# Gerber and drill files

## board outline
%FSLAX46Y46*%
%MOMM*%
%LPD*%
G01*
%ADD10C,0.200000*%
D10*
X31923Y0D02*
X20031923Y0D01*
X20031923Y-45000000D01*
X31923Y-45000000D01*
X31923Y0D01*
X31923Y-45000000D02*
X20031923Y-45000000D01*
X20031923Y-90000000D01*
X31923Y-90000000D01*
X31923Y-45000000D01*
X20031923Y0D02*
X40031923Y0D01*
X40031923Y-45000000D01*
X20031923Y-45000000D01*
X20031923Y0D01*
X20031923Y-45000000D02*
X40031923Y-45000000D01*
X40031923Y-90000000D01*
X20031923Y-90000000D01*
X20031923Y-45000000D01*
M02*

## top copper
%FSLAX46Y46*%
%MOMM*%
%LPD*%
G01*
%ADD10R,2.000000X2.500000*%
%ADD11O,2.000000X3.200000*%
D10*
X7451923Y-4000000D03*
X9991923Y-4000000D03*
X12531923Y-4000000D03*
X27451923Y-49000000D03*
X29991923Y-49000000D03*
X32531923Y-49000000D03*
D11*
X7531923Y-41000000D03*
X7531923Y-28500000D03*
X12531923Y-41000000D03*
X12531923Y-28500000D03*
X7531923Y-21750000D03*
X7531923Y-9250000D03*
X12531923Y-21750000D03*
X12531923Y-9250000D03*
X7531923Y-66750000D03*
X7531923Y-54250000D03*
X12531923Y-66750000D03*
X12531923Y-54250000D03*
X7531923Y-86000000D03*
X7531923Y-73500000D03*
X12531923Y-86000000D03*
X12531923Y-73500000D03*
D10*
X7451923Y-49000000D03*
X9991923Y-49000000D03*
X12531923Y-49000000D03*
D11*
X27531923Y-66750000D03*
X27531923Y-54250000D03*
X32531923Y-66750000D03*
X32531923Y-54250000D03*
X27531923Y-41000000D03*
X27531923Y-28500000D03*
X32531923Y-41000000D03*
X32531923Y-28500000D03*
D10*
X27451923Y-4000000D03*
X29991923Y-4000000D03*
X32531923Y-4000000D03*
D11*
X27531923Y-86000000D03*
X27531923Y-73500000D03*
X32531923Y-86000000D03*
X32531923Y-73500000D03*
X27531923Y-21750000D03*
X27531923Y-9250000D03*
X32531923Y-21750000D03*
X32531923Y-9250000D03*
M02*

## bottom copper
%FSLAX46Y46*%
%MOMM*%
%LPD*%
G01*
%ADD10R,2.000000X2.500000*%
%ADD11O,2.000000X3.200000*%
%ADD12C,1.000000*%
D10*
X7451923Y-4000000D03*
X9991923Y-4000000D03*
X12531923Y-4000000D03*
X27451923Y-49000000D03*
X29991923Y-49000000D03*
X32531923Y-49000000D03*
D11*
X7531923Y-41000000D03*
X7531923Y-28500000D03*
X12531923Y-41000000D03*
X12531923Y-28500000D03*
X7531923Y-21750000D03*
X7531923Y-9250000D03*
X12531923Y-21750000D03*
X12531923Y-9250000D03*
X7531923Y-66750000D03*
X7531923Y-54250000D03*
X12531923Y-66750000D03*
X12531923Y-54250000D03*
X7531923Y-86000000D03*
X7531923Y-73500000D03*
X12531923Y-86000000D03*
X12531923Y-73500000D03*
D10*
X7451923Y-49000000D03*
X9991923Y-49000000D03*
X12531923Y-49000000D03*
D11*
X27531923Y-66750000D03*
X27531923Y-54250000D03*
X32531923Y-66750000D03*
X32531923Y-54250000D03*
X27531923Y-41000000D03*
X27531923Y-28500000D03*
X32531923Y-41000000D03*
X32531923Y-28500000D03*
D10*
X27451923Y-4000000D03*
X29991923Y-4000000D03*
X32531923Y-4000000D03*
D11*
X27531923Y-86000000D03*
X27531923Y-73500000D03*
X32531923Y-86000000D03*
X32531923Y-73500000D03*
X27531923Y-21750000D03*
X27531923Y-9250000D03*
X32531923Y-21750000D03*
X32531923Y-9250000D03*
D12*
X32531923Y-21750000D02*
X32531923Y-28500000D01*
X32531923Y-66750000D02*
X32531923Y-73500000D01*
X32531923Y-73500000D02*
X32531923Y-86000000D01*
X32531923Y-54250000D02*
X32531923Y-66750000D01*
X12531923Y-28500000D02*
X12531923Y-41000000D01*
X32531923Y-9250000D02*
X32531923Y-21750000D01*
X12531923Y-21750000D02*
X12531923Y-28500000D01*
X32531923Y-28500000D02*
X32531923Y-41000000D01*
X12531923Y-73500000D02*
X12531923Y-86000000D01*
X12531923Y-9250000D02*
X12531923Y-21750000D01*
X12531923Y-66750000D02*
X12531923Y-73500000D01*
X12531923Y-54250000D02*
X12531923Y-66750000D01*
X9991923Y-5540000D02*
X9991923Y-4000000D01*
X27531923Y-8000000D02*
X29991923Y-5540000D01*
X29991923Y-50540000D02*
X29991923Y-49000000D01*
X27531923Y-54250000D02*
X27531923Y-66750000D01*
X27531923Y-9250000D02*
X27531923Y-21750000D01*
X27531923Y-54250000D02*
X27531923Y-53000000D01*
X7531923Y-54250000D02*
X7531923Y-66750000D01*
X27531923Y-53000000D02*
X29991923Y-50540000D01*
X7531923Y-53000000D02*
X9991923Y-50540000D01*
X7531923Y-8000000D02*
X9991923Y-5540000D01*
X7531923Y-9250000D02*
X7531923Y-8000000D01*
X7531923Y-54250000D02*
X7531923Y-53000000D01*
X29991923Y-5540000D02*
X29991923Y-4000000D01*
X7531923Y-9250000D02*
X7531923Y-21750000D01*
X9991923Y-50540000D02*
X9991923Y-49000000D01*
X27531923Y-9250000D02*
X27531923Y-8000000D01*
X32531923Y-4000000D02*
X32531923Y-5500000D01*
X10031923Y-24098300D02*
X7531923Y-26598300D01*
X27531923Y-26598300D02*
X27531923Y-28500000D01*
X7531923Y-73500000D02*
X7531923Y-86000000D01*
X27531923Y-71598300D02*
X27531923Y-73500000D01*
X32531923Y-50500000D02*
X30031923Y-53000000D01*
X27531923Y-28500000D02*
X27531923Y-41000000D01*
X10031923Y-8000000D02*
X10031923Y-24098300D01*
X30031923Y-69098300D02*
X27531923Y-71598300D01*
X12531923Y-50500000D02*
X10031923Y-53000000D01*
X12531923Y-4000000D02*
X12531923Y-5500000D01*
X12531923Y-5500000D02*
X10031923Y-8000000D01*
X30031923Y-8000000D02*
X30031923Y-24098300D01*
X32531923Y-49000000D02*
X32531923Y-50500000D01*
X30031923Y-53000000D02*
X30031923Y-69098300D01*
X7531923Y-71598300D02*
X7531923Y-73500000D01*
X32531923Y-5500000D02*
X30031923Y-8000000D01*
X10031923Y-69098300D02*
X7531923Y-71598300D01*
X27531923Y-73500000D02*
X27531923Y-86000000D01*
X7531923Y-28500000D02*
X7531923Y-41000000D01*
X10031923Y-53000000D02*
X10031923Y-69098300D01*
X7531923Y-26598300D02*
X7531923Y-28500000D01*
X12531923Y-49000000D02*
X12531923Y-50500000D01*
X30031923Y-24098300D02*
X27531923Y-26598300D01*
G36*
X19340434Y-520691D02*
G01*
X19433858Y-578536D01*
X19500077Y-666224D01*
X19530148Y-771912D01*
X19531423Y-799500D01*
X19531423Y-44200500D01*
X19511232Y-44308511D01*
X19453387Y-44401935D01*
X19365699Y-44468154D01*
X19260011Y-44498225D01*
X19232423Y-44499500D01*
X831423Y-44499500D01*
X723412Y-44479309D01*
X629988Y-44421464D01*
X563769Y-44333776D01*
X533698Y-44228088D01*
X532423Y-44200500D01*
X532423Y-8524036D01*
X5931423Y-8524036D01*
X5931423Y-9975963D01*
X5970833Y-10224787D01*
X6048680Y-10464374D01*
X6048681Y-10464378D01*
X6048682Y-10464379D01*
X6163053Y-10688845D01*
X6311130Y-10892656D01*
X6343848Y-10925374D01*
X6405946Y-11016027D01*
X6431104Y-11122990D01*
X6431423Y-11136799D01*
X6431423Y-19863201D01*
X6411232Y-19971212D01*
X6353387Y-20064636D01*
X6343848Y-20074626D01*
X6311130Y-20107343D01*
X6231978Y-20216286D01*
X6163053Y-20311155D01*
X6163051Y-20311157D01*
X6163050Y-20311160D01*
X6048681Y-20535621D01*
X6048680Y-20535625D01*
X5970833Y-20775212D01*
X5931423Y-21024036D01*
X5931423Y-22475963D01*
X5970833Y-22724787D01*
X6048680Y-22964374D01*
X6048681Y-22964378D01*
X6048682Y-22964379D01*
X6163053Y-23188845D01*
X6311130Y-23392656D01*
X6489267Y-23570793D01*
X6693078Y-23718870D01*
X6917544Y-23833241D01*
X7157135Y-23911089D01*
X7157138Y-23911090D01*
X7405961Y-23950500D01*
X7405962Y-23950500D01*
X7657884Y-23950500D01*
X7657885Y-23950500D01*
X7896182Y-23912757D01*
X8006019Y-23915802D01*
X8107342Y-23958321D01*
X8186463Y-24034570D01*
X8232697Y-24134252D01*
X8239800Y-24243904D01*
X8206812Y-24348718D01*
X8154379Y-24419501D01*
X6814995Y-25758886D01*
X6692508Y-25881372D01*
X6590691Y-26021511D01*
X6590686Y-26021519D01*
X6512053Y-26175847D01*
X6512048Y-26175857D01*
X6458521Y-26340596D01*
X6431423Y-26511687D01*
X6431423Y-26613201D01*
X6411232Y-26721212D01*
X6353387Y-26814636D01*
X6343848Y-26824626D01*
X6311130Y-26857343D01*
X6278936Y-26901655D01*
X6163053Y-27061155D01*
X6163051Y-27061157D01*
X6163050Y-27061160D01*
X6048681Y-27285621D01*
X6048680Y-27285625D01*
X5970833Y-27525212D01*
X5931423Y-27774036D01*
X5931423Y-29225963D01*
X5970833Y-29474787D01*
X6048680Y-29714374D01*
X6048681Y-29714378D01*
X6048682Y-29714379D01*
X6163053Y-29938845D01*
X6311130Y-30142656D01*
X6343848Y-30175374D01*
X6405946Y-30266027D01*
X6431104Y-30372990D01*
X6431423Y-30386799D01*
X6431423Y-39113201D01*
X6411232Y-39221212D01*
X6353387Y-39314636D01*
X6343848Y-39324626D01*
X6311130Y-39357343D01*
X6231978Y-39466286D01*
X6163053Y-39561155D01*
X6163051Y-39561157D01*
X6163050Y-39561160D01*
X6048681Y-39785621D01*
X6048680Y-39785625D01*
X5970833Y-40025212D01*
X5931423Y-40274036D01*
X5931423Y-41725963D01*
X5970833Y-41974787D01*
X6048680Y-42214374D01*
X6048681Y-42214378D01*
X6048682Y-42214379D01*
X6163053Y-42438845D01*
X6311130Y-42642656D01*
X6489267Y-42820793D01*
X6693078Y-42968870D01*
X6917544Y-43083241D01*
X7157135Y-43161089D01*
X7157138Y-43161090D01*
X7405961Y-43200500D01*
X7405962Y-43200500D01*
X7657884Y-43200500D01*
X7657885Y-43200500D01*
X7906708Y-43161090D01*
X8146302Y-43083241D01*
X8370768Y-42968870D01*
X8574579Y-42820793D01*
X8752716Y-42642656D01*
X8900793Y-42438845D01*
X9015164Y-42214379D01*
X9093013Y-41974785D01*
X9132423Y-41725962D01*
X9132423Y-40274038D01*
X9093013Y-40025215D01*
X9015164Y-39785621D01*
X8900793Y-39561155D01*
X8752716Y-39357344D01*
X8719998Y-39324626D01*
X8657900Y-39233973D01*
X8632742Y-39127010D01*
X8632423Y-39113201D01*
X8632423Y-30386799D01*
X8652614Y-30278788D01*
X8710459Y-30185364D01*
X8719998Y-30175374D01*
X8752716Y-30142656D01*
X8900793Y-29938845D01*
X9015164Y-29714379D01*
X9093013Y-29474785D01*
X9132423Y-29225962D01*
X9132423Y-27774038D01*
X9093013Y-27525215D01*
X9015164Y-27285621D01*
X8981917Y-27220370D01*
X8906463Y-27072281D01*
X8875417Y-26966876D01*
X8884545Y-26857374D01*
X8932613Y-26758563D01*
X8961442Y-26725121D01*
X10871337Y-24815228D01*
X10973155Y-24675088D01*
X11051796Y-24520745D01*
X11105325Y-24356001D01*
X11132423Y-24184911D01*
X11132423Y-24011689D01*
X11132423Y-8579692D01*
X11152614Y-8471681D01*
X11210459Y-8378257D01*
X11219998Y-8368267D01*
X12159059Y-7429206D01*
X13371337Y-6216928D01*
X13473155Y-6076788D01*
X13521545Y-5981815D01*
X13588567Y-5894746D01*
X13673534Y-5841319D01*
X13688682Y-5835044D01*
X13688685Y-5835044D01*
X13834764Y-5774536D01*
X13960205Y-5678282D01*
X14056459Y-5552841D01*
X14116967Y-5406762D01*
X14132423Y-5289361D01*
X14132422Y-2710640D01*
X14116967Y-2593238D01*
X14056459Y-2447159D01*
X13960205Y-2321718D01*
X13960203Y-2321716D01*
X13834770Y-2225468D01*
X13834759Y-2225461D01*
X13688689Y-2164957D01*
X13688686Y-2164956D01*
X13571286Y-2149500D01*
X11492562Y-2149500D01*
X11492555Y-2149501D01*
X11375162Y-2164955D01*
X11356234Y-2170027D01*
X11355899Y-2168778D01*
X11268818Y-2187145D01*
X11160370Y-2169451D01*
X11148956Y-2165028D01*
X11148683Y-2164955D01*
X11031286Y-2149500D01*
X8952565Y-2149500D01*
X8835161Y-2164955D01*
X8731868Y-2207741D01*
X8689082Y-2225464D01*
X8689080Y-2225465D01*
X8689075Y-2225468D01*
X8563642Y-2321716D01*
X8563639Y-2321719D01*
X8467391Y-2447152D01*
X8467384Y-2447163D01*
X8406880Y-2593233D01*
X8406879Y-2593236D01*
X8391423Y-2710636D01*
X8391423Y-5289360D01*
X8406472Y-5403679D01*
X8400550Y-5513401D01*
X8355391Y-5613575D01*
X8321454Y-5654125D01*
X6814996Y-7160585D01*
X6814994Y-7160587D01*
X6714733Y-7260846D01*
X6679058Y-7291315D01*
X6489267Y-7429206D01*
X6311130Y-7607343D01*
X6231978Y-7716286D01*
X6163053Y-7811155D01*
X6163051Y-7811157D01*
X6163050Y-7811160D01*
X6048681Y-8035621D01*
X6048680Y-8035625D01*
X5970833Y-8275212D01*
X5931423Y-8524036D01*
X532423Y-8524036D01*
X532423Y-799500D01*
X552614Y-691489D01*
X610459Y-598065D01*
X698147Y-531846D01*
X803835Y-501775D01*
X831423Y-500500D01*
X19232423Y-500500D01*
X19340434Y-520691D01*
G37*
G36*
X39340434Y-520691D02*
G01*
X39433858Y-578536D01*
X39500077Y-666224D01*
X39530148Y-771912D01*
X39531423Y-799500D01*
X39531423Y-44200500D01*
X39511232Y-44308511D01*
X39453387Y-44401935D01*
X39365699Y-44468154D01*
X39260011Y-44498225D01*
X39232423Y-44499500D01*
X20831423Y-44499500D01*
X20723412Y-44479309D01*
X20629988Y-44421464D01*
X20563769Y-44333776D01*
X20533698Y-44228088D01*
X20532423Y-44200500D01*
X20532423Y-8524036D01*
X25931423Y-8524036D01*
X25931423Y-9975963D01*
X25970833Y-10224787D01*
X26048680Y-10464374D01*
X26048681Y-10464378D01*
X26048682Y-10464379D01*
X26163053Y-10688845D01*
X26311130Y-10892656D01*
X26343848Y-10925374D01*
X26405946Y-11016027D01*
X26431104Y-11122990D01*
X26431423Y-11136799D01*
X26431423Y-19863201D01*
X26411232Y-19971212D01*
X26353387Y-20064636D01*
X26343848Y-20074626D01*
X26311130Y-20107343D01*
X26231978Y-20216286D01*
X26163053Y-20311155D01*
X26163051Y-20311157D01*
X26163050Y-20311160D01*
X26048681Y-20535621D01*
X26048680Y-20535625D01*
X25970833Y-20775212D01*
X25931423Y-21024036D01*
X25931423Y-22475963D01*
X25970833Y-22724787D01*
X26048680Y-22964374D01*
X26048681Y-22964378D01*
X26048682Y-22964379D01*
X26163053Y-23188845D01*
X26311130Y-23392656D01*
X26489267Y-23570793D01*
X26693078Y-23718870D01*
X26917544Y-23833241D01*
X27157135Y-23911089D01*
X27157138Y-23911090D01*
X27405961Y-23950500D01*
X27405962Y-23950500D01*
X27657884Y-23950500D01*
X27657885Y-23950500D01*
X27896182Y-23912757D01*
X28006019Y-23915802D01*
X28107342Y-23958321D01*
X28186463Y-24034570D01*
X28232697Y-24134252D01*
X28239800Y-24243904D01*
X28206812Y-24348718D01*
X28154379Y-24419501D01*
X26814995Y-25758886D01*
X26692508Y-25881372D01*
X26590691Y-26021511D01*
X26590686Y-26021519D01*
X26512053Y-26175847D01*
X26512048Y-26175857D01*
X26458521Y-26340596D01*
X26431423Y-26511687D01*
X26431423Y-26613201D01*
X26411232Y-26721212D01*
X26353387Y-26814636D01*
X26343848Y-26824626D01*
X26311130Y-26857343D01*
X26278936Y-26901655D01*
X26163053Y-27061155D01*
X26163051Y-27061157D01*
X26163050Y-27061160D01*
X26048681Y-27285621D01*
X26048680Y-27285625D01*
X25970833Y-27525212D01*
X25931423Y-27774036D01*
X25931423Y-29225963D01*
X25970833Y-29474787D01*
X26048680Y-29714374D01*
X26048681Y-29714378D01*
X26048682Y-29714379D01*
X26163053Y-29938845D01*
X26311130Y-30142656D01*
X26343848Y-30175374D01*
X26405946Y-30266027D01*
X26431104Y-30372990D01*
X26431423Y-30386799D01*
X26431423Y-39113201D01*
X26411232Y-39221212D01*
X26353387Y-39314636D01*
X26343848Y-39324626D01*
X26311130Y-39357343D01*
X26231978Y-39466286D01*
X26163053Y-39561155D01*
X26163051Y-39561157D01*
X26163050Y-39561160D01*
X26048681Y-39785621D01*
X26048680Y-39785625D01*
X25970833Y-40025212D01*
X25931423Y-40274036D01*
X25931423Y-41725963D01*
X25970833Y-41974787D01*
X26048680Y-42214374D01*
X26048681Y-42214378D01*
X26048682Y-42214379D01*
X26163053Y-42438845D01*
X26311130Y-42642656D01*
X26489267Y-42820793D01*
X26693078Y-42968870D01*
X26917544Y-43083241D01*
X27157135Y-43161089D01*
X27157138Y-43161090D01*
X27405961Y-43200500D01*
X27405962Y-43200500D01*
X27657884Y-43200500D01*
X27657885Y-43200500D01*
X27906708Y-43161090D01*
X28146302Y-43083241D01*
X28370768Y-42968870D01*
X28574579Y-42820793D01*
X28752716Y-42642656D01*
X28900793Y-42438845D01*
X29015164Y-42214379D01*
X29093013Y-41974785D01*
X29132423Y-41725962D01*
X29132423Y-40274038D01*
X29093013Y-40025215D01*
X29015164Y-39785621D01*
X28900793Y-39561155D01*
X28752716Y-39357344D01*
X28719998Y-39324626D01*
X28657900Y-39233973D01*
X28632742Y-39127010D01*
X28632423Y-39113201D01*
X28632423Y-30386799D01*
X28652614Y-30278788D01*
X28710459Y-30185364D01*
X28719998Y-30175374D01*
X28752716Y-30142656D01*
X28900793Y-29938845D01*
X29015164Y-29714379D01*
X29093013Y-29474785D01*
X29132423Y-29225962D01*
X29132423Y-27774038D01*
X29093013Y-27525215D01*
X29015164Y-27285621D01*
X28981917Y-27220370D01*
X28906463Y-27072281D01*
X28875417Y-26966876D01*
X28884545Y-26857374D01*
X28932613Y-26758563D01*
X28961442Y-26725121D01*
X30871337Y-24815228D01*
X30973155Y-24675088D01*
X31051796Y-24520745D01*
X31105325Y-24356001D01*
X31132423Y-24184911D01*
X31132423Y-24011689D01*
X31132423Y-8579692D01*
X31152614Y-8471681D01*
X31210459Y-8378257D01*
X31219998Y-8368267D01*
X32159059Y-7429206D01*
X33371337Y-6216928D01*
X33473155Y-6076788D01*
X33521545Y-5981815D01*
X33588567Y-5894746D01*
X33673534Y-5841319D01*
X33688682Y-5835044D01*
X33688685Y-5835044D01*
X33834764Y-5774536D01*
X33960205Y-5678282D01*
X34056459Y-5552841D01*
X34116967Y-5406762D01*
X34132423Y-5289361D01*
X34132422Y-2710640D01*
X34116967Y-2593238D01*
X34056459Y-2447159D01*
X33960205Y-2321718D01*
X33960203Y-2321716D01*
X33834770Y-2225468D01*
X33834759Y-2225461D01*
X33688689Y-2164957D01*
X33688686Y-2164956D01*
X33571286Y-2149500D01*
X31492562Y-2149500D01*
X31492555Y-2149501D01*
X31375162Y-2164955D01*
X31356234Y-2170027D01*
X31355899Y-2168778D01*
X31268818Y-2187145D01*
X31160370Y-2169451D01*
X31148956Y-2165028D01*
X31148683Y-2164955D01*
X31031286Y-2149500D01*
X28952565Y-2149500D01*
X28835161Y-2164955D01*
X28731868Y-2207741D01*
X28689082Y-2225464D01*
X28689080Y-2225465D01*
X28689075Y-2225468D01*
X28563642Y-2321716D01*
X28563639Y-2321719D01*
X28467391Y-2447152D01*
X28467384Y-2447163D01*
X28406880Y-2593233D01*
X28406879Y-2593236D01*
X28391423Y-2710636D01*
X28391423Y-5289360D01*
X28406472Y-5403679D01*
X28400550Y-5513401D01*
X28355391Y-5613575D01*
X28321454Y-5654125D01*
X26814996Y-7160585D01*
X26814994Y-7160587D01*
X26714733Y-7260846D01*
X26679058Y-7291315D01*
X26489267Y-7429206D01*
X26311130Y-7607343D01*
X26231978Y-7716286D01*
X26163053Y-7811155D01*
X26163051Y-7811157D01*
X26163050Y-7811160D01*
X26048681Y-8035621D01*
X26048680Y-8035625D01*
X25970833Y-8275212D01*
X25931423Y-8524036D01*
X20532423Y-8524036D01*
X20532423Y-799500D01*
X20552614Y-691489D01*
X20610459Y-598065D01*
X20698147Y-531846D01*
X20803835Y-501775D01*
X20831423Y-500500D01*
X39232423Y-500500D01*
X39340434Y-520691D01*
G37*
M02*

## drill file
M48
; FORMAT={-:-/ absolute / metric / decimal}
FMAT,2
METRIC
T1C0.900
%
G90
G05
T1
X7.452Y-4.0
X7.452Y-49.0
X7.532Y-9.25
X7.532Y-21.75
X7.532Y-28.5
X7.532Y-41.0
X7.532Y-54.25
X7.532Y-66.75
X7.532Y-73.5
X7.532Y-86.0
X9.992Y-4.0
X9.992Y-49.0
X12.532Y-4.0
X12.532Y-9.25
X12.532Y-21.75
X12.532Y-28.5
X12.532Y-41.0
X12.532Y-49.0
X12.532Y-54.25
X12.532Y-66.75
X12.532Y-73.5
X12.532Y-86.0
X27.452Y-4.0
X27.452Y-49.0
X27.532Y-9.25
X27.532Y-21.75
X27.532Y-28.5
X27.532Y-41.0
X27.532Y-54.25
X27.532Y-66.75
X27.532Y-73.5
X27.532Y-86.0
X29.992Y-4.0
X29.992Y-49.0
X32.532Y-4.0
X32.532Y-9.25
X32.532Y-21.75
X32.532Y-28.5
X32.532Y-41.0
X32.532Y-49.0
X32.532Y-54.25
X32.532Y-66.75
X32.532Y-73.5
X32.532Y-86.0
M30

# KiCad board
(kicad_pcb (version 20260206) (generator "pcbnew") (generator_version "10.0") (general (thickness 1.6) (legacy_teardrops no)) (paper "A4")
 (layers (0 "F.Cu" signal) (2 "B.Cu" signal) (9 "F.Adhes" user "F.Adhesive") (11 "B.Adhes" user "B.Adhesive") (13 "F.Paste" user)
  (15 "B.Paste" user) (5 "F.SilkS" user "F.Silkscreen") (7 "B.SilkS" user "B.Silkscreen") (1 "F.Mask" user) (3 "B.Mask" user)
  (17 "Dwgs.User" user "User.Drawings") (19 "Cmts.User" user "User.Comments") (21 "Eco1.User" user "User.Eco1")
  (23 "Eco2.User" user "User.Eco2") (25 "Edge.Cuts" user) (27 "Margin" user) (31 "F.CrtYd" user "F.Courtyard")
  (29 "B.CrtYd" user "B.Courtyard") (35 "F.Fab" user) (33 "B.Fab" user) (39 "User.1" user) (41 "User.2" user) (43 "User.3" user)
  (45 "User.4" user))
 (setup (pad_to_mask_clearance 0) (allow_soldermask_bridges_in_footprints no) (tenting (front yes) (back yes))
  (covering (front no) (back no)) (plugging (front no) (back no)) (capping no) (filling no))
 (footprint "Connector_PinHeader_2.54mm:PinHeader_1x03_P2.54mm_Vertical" (layer "F.Cu") (at 7.451923 4 90)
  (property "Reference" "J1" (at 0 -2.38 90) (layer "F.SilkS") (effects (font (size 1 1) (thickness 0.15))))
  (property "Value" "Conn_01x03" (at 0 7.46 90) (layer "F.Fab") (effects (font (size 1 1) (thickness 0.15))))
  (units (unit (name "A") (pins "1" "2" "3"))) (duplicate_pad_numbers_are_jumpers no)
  (pad "1" thru_hole rect (at 0 0 90) (size 2.5 2) (drill 0.9) (layers "*.Cu" "*.Mask") (remove_unused_layers no) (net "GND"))
  (pad "2" thru_hole rect (at 0 2.54 90) (size 2.5 2) (drill 0.9) (layers "*.Cu" "*.Mask") (remove_unused_layers no) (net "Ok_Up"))
  (pad "3" thru_hole rect (at 0 5.08 90) (size 2.5 2) (drill 0.9) (layers "*.Cu" "*.Mask") (remove_unused_layers no) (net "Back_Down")))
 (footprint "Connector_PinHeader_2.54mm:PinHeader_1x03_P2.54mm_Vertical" (layer "F.Cu") (at 27.451923 49 90)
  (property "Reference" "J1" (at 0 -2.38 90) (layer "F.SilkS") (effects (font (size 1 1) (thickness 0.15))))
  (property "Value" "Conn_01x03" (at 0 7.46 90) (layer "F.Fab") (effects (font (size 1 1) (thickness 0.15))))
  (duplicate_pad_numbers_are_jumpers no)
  (pad "1" thru_hole rect (at 0 0 90) (size 2.5 2) (drill 0.9) (layers "*.Cu" "*.Mask") (remove_unused_layers no) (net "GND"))
  (pad "2" thru_hole rect (at 0 2.54 90) (size 2.5 2) (drill 0.9) (layers "*.Cu" "*.Mask") (remove_unused_layers no) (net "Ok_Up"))
  (pad "3" thru_hole rect (at 0 5.08 90) (size 2.5 2) (drill 0.9) (layers "*.Cu" "*.Mask") (remove_unused_layers no) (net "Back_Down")))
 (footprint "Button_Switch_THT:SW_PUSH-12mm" (layer "F.Cu") (at 7.531923 41 90)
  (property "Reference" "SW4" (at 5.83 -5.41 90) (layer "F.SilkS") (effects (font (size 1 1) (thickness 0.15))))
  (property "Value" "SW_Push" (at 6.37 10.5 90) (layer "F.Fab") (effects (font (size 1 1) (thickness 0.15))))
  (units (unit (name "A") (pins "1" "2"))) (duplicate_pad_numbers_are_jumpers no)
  (pad "1" thru_hole oval (at 0 0 90) (size 3.2 2) (drill 0.9) (layers "*.Cu" "*.Mask") (remove_unused_layers no) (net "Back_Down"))
  (pad "1" thru_hole oval (at 12.5 0 90) (size 3.2 2) (drill 0.9) (layers "*.Cu" "*.Mask") (remove_unused_layers no) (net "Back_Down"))
  (pad "2" thru_hole oval (at 0 5 90) (size 3.2 2) (drill 0.9) (layers "*.Cu" "*.Mask") (remove_unused_layers no) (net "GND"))
  (pad "2" thru_hole oval (at 12.5 5 90) (size 3.2 2) (drill 0.9) (layers "*.Cu" "*.Mask") (remove_unused_layers no) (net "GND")))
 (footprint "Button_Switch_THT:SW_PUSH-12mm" (layer "F.Cu") (at 7.531923 21.75 90)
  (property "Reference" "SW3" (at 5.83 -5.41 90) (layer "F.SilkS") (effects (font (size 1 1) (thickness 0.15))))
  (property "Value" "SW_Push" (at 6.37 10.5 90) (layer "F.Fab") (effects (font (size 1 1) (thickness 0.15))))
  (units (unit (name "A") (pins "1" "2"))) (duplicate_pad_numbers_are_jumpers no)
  (pad "1" thru_hole oval (at 0 0 90) (size 3.2 2) (drill 0.9) (layers "*.Cu" "*.Mask") (remove_unused_layers no) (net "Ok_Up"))
  (pad "1" thru_hole oval (at 12.5 0 90) (size 3.2 2) (drill 0.9) (layers "*.Cu" "*.Mask") (remove_unused_layers no) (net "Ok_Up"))
  (pad "2" thru_hole oval (at 0 5 90) (size 3.2 2) (drill 0.9) (layers "*.Cu" "*.Mask") (remove_unused_layers no) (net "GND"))
  (pad "2" thru_hole oval (at 12.5 5 90) (size 3.2 2) (drill 0.9) (layers "*.Cu" "*.Mask") (remove_unused_layers no) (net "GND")))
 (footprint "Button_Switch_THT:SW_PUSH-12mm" (layer "F.Cu") (at 7.531923 66.75 90)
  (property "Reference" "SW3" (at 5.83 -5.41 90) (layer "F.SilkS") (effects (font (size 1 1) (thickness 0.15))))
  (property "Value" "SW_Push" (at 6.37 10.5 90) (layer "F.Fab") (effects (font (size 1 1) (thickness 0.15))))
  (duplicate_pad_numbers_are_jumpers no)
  (pad "1" thru_hole oval (at 0 0 90) (size 3.2 2) (drill 0.9) (layers "*.Cu" "*.Mask") (remove_unused_layers no) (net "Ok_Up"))
  (pad "1" thru_hole oval (at 12.5 0 90) (size 3.2 2) (drill 0.9) (layers "*.Cu" "*.Mask") (remove_unused_layers no) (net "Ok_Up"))
  (pad "2" thru_hole oval (at 0 5 90) (size 3.2 2) (drill 0.9) (layers "*.Cu" "*.Mask") (remove_unused_layers no) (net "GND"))
  (pad "2" thru_hole oval (at 12.5 5 90) (size 3.2 2) (drill 0.9) (layers "*.Cu" "*.Mask") (remove_unused_layers no) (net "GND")))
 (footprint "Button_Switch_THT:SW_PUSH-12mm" (layer "F.Cu") (at 7.531923 86 90)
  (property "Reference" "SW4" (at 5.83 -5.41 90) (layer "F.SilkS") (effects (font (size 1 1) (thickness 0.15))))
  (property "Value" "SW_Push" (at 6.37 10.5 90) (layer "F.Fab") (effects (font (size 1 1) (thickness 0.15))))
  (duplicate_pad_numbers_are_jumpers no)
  (pad "1" thru_hole oval (at 0 0 90) (size 3.2 2) (drill 0.9) (layers "*.Cu" "*.Mask") (remove_unused_layers no) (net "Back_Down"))
  (pad "1" thru_hole oval (at 12.5 0 90) (size 3.2 2) (drill 0.9) (layers "*.Cu" "*.Mask") (remove_unused_layers no) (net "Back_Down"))
  (pad "2" thru_hole oval (at 0 5 90) (size 3.2 2) (drill 0.9) (layers "*.Cu" "*.Mask") (remove_unused_layers no) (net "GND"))
  (pad "2" thru_hole oval (at 12.5 5 90) (size 3.2 2) (drill 0.9) (layers "*.Cu" "*.Mask") (remove_unused_layers no) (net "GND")))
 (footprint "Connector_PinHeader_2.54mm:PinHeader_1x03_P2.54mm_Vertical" (layer "F.Cu") (at 7.451923 49 90)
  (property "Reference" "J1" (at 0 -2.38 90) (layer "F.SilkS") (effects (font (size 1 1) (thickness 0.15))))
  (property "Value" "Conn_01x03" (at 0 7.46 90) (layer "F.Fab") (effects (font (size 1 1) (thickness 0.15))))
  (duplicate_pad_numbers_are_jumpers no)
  (pad "1" thru_hole rect (at 0 0 90) (size 2.5 2) (drill 0.9) (layers "*.Cu" "*.Mask") (remove_unused_layers no) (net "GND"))
  (pad "2" thru_hole rect (at 0 2.54 90) (size 2.5 2) (drill 0.9) (layers "*.Cu" "*.Mask") (remove_unused_layers no) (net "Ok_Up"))
  (pad "3" thru_hole rect (at 0 5.08 90) (size 2.5 2) (drill 0.9) (layers "*.Cu" "*.Mask") (remove_unused_layers no) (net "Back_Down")))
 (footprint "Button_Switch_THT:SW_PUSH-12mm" (layer "F.Cu") (at 27.531923 66.75 90)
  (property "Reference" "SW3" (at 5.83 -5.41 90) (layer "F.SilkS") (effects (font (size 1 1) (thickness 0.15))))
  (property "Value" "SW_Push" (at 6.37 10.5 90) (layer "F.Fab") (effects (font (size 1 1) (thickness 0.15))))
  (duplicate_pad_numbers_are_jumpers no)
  (pad "1" thru_hole oval (at 0 0 90) (size 3.2 2) (drill 0.9) (layers "*.Cu" "*.Mask") (remove_unused_layers no) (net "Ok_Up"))
  (pad "1" thru_hole oval (at 12.5 0 90) (size 3.2 2) (drill 0.9) (layers "*.Cu" "*.Mask") (remove_unused_layers no) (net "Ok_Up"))
  (pad "2" thru_hole oval (at 0 5 90) (size 3.2 2) (drill 0.9) (layers "*.Cu" "*.Mask") (remove_unused_layers no) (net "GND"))
  (pad "2" thru_hole oval (at 12.5 5 90) (size 3.2 2) (drill 0.9) (layers "*.Cu" "*.Mask") (remove_unused_layers no) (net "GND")))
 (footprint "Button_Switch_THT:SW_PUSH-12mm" (layer "F.Cu") (at 27.531923 41 90)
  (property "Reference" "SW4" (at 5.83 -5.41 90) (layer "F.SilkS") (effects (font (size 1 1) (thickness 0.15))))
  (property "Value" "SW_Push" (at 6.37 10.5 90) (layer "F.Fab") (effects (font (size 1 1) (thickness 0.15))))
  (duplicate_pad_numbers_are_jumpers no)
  (pad "1" thru_hole oval (at 0 0 90) (size 3.2 2) (drill 0.9) (layers "*.Cu" "*.Mask") (remove_unused_layers no) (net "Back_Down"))
  (pad "1" thru_hole oval (at 12.5 0 90) (size 3.2 2) (drill 0.9) (layers "*.Cu" "*.Mask") (remove_unused_layers no) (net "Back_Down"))
  (pad "2" thru_hole oval (at 0 5 90) (size 3.2 2) (drill 0.9) (layers "*.Cu" "*.Mask") (remove_unused_layers no) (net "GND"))
  (pad "2" thru_hole oval (at 12.5 5 90) (size 3.2 2) (drill 0.9) (layers "*.Cu" "*.Mask") (remove_unused_layers no) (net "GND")))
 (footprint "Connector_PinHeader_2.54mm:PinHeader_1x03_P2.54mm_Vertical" (layer "F.Cu") (at 27.451923 4 90)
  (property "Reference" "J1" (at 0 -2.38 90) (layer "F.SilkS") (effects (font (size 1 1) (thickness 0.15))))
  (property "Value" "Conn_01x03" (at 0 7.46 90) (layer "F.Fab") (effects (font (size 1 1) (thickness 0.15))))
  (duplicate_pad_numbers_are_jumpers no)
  (pad "1" thru_hole rect (at 0 0 90) (size 2.5 2) (drill 0.9) (layers "*.Cu" "*.Mask") (remove_unused_layers no) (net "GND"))
  (pad "2" thru_hole rect (at 0 2.54 90) (size 2.5 2) (drill 0.9) (layers "*.Cu" "*.Mask") (remove_unused_layers no) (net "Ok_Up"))
  (pad "3" thru_hole rect (at 0 5.08 90) (size 2.5 2) (drill 0.9) (layers "*.Cu" "*.Mask") (remove_unused_layers no) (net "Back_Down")))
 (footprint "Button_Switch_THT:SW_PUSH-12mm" (layer "F.Cu") (at 27.531923 86 90)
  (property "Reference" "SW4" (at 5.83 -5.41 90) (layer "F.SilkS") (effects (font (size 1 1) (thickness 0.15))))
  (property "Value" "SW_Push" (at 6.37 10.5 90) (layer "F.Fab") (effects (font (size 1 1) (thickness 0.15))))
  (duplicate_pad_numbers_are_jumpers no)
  (pad "1" thru_hole oval (at 0 0 90) (size 3.2 2) (drill 0.9) (layers "*.Cu" "*.Mask") (remove_unused_layers no) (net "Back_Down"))
  (pad "1" thru_hole oval (at 12.5 0 90) (size 3.2 2) (drill 0.9) (layers "*.Cu" "*.Mask") (remove_unused_layers no) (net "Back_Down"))
  (pad "2" thru_hole oval (at 0 5 90) (size 3.2 2) (drill 0.9) (layers "*.Cu" "*.Mask") (remove_unused_layers no) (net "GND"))
  (pad "2" thru_hole oval (at 12.5 5 90) (size 3.2 2) (drill 0.9) (layers "*.Cu" "*.Mask") (remove_unused_layers no) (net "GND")))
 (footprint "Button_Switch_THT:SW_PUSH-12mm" (layer "F.Cu") (at 27.531923 21.75 90)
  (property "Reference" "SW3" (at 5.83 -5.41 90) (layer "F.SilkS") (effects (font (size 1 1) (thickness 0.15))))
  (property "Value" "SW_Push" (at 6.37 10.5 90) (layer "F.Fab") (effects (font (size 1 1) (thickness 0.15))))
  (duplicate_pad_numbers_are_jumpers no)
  (pad "1" thru_hole oval (at 0 0 90) (size 3.2 2) (drill 0.9) (layers "*.Cu" "*.Mask") (remove_unused_layers no) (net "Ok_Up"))
  (pad "1" thru_hole oval (at 12.5 0 90) (size 3.2 2) (drill 0.9) (layers "*.Cu" "*.Mask") (remove_unused_layers no) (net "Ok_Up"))
  (pad "2" thru_hole oval (at 0 5 90) (size 3.2 2) (drill 0.9) (layers "*.Cu" "*.Mask") (remove_unused_layers no) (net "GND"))
  (pad "2" thru_hole oval (at 12.5 5 90) (size 3.2 2) (drill 0.9) (layers "*.Cu" "*.Mask") (remove_unused_layers no) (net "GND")))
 (gr_rect (start 0.031923 0) (end 20.031923 45) (stroke (width 0.2) (type default)) (fill no) (layer "Edge.Cuts"))
 (gr_rect (start 0.031923 45) (end 20.031923 90) (stroke (width 0.2) (type default)) (fill no) (layer "Edge.Cuts"))
 (gr_rect (start 20.031923 0) (end 40.031923 45) (stroke (width 0.2) (type default)) (fill no) (layer "Edge.Cuts"))
 (gr_rect (start 20.031923 45) (end 40.031923 90) (stroke (width 0.2) (type default)) (fill no) (layer "Edge.Cuts"))
 (segment (start 32.531923 21.75) (end 32.531923 28.5) (width 1) (layer "B.Cu") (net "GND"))
 (segment (start 32.531923 66.75) (end 32.531923 73.5) (width 1) (layer "B.Cu") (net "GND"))
 (segment (start 32.531923 73.5) (end 32.531923 86) (width 1) (layer "B.Cu") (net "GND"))
 (segment (start 32.531923 54.25) (end 32.531923 66.75) (width 1) (layer "B.Cu") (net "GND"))
 (segment (start 12.531923 28.5) (end 12.531923 41) (width 1) (layer "B.Cu") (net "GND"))
 (segment (start 32.531923 9.25) (end 32.531923 21.75) (width 1) (layer "B.Cu") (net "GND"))
 (segment (start 12.531923 21.75) (end 12.531923 28.5) (width 1) (layer "B.Cu") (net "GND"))
 (segment (start 32.531923 28.5) (end 32.531923 41) (width 1) (layer "B.Cu") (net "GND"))
 (segment (start 12.531923 73.5) (end 12.531923 86) (width 1) (layer "B.Cu") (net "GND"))
 (segment (start 12.531923 9.25) (end 12.531923 21.75) (width 1) (layer "B.Cu") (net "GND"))
 (segment (start 12.531923 66.75) (end 12.531923 73.5) (width 1) (layer "B.Cu") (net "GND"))
 (segment (start 12.531923 54.25) (end 12.531923 66.75) (width 1) (layer "B.Cu") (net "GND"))
 (segment (start 9.991923 5.54) (end 9.991923 4) (width 1) (layer "B.Cu") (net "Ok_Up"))
 (segment (start 27.531923 8) (end 29.991923 5.54) (width 1) (layer "B.Cu") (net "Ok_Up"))
 (segment (start 29.991923 50.54) (end 29.991923 49) (width 1) (layer "B.Cu") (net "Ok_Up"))
 (segment (start 27.531923 54.25) (end 27.531923 66.75) (width 1) (layer "B.Cu") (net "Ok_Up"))
 (segment (start 27.531923 9.25) (end 27.531923 21.75) (width 1) (layer "B.Cu") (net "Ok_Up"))
 (segment (start 27.531923 54.25) (end 27.531923 53) (width 1) (layer "B.Cu") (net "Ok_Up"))
 (segment (start 7.531923 54.25) (end 7.531923 66.75) (width 1) (layer "B.Cu") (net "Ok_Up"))
 (segment (start 27.531923 53) (end 29.991923 50.54) (width 1) (layer "B.Cu") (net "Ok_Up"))
 (segment (start 7.531923 53) (end 9.991923 50.54) (width 1) (layer "B.Cu") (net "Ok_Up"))
 (segment (start 7.531923 8) (end 9.991923 5.54) (width 1) (layer "B.Cu") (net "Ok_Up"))
 (segment (start 7.531923 9.25) (end 7.531923 8) (width 1) (layer "B.Cu") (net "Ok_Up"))
 (segment (start 7.531923 54.25) (end 7.531923 53) (width 1) (layer "B.Cu") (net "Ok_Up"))
 (segment (start 29.991923 5.54) (end 29.991923 4) (width 1) (layer "B.Cu") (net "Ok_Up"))
 (segment (start 7.531923 9.25) (end 7.531923 21.75) (width 1) (layer "B.Cu") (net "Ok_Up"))
 (segment (start 9.991923 50.54) (end 9.991923 49) (width 1) (layer "B.Cu") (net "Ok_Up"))
 (segment (start 27.531923 9.25) (end 27.531923 8) (width 1) (layer "B.Cu") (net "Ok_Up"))
 (segment (start 32.531923 4) (end 32.531923 5.5) (width 1) (layer "B.Cu") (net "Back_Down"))
 (segment (start 10.031923 24.0983) (end 7.531923 26.5983) (width 1) (layer "B.Cu") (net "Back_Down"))
 (segment (start 27.531923 26.5983) (end 27.531923 28.5) (width 1) (layer "B.Cu") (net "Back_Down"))
 (segment (start 7.531923 73.5) (end 7.531923 86) (width 1) (layer "B.Cu") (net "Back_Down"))
 (segment (start 27.531923 71.5983) (end 27.531923 73.5) (width 1) (layer "B.Cu") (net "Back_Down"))
 (segment (start 32.531923 50.5) (end 30.031923 53) (width 1) (layer "B.Cu") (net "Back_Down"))
 (segment (start 27.531923 28.5) (end 27.531923 41) (width 1) (layer "B.Cu") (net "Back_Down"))
 (segment (start 10.031923 8) (end 10.031923 24.0983) (width 1) (layer "B.Cu") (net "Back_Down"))
 (segment (start 30.031923 69.0983) (end 27.531923 71.5983) (width 1) (layer "B.Cu") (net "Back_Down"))
 (segment (start 12.531923 50.5) (end 10.031923 53) (width 1) (layer "B.Cu") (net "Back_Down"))
 (segment (start 12.531923 4) (end 12.531923 5.5) (width 1) (layer "B.Cu") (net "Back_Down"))
 (segment (start 12.531923 5.5) (end 10.031923 8) (width 1) (layer "B.Cu") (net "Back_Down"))
 (segment (start 30.031923 8) (end 30.031923 24.0983) (width 1) (layer "B.Cu") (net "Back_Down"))
 (segment (start 32.531923 49) (end 32.531923 50.5) (width 1) (layer "B.Cu") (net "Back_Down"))
 (segment (start 30.031923 53) (end 30.031923 69.0983) (width 1) (layer "B.Cu") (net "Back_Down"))
 (segment (start 7.531923 71.5983) (end 7.531923 73.5) (width 1) (layer "B.Cu") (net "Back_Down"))
 (segment (start 32.531923 5.5) (end 30.031923 8) (width 1) (layer "B.Cu") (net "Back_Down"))
 (segment (start 10.031923 69.0983) (end 7.531923 71.5983) (width 1) (layer "B.Cu") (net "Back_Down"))
 (segment (start 27.531923 73.5) (end 27.531923 86) (width 1) (layer "B.Cu") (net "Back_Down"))
 (segment (start 7.531923 28.5) (end 7.531923 41) (width 1) (layer "B.Cu") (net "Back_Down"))
 (segment (start 10.031923 53) (end 10.031923 69.0983) (width 1) (layer "B.Cu") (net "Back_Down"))
 (segment (start 7.531923 26.5983) (end 7.531923 28.5) (width 1) (layer "B.Cu") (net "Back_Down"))
 (segment (start 12.531923 49) (end 12.531923 50.5) (width 1) (layer "B.Cu") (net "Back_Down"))
 (segment (start 30.031923 24.0983) (end 27.531923 26.5983) (width 1) (layer "B.Cu") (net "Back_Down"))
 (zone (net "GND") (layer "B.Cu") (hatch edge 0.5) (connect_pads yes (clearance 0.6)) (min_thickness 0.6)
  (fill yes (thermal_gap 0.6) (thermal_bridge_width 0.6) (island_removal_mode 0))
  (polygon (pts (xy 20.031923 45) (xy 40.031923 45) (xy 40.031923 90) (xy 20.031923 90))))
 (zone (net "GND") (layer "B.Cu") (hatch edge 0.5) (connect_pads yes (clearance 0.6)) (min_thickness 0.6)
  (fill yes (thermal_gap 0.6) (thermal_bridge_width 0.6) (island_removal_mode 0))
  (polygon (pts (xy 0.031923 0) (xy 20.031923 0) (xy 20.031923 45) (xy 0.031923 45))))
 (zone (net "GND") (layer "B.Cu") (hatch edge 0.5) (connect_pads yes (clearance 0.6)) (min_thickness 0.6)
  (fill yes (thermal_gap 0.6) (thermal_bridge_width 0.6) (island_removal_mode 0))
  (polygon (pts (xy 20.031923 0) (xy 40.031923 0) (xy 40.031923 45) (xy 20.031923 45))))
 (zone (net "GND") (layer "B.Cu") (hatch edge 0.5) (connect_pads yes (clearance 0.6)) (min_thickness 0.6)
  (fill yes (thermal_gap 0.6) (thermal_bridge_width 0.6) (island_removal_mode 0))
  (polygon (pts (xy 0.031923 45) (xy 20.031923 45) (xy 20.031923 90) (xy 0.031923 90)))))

